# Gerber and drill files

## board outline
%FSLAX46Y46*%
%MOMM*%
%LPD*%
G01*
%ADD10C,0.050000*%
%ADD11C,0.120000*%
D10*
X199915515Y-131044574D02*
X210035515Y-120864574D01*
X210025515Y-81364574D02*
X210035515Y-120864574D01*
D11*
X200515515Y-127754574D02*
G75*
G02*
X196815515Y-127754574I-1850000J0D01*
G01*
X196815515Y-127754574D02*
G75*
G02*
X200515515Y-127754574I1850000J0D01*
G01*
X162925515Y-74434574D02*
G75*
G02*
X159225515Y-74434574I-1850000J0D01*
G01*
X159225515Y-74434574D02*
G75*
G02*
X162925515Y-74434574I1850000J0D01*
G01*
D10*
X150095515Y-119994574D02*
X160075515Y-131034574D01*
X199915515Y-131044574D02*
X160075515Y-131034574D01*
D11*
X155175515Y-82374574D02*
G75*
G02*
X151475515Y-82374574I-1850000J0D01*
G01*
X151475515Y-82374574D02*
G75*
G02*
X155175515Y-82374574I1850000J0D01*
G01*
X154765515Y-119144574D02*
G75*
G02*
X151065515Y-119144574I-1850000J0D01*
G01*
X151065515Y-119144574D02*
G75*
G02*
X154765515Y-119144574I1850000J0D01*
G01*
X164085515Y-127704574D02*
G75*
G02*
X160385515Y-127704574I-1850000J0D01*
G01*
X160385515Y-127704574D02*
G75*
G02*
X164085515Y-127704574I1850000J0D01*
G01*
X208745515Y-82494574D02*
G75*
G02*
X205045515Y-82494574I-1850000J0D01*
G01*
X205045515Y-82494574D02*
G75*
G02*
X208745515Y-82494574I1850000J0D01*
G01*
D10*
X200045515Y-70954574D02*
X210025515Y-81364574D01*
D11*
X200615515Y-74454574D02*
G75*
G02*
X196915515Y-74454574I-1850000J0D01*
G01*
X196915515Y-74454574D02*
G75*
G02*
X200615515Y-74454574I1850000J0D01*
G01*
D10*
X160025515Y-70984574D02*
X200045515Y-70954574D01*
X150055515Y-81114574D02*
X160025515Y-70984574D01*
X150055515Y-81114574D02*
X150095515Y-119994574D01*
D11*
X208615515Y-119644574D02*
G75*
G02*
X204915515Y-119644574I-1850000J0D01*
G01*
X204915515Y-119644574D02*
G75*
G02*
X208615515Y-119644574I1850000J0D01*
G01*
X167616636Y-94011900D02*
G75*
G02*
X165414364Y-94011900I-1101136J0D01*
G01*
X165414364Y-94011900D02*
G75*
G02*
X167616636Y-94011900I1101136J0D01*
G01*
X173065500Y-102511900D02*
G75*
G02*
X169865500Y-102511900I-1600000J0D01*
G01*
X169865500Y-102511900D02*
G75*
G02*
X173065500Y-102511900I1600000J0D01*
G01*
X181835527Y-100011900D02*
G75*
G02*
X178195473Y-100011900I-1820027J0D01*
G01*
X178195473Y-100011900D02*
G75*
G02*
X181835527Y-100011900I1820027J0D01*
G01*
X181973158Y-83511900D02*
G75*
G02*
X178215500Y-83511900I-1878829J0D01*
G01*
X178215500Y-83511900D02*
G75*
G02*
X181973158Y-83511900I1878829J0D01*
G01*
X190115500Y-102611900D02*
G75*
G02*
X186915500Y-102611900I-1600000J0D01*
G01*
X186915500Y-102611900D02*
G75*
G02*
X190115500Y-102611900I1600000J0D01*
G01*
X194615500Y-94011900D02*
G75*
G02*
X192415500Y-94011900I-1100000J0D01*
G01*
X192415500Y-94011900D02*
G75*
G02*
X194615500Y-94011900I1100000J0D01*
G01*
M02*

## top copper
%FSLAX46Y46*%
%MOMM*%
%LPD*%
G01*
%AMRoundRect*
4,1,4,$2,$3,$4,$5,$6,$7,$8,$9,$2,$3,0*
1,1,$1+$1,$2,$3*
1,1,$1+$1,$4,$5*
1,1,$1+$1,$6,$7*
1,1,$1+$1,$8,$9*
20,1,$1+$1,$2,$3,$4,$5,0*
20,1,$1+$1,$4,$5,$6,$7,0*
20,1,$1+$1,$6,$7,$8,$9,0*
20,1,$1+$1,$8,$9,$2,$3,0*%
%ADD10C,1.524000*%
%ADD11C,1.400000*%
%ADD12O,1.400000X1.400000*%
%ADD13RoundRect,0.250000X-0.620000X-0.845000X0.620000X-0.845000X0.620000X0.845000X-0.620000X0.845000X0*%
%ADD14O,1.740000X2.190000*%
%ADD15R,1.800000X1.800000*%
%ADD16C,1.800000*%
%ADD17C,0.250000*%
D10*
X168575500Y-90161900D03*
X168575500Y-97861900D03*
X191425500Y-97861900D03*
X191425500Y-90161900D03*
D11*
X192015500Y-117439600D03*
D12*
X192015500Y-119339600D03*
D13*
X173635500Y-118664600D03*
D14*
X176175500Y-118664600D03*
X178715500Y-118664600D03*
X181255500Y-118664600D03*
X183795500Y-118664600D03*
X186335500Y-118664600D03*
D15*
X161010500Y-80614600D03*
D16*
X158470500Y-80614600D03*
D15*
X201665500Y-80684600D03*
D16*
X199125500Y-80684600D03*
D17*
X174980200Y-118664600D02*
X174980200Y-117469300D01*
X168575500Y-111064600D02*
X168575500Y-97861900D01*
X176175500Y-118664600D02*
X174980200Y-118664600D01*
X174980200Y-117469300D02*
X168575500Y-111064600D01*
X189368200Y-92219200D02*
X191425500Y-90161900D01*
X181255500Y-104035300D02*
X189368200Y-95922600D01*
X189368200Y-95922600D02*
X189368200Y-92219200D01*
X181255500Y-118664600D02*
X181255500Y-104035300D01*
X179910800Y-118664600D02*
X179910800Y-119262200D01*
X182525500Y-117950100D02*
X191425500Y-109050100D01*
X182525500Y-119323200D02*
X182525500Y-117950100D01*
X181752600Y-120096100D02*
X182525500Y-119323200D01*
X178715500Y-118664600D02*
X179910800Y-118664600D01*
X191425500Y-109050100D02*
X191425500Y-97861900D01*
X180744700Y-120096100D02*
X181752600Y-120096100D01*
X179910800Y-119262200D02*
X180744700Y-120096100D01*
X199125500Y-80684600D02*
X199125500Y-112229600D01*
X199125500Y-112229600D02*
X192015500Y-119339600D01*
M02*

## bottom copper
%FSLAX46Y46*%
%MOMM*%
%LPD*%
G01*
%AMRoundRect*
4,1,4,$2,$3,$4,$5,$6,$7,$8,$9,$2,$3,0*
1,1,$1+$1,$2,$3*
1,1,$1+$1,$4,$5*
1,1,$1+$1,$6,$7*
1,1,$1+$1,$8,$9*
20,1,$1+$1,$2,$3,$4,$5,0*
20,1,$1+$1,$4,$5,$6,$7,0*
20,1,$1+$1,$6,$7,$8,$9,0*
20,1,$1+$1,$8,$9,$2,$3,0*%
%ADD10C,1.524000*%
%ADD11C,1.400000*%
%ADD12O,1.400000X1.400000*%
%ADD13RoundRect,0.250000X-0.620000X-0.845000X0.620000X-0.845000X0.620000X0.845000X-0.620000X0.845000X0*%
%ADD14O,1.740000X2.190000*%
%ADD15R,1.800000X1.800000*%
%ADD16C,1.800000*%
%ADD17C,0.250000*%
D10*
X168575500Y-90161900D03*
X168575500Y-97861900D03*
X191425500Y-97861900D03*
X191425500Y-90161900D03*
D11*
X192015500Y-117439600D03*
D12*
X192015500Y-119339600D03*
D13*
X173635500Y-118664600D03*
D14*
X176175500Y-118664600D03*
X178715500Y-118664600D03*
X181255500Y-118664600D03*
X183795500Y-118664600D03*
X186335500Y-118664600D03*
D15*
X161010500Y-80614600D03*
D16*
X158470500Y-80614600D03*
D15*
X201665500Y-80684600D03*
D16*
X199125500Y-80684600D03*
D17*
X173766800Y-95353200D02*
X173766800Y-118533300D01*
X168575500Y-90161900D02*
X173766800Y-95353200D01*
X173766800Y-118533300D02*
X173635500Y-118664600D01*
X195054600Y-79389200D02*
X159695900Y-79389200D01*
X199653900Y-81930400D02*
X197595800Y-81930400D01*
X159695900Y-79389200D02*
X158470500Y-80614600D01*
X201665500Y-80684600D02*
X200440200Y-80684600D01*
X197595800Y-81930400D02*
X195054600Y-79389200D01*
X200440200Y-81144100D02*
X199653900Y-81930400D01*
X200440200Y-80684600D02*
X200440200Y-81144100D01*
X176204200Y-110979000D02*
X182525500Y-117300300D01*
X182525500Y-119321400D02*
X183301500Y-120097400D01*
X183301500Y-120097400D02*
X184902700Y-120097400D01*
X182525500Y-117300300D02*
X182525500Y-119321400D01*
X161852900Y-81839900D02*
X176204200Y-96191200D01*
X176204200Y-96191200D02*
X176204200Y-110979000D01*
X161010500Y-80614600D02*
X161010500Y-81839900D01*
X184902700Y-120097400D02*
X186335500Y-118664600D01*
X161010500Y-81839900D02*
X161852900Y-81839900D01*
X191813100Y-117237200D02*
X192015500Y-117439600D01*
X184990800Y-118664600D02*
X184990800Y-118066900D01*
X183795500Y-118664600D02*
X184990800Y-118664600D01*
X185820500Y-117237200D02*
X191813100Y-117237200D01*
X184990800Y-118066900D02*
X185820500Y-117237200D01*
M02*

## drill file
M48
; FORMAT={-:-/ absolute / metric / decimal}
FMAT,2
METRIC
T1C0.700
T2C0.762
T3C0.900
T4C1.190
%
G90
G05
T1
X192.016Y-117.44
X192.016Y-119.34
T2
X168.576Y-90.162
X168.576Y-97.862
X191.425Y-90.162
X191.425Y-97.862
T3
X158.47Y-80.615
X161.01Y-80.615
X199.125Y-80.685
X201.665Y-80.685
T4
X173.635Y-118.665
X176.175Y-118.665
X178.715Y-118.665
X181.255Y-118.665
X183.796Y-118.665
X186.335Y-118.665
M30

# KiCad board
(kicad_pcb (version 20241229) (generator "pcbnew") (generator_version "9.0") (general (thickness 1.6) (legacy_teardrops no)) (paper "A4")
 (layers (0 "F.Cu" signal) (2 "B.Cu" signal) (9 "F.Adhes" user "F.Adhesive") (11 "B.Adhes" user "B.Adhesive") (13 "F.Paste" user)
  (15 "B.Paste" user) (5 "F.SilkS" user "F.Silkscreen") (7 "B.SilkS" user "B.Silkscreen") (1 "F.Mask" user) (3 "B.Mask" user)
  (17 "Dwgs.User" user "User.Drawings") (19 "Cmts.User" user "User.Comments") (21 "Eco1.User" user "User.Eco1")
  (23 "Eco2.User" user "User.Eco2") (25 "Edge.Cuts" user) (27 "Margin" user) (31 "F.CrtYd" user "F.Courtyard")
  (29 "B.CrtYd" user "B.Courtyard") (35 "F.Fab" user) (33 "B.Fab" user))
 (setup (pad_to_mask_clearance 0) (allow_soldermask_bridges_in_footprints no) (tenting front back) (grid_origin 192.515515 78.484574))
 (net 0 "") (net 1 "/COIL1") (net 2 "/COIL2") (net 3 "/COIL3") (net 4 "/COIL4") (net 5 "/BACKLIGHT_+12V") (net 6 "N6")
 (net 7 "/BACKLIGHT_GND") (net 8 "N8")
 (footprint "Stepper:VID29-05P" (layer "F.Cu") (at 180.0155 94.0119)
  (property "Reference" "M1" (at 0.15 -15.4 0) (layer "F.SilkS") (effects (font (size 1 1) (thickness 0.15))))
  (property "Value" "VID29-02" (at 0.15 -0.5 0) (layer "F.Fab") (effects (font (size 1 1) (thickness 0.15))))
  (fp_circle (center -13.5 0) (end -12.65 0.7) (stroke (width 0.12) (type solid)) (fill no) (layer "Edge.Cuts"))
  (fp_circle (center -8.55 8.5) (end -6.95 8.5) (stroke (width 0.12) (type solid)) (fill no) (layer "Edge.Cuts"))
  (fp_circle (center 0 6) (end 1.45 7.1) (stroke (width 0.12) (type solid)) (fill no) (layer "Edge.Cuts"))
  (fp_circle (center 0.078829 -10.5) (end 1.778829 -9.7) (stroke (width 0.12) (type solid)) (fill no) (layer "Edge.Cuts"))
  (fp_circle (center 8.5 8.6) (end 10.1 8.6) (stroke (width 0.12) (type solid)) (fill no) (layer "Edge.Cuts"))
  (fp_circle (center 13.5 0) (end 14.6 0) (stroke (width 0.12) (type solid)) (fill no) (layer "Edge.Cuts"))
  (pad "1" thru_hole circle (at -11.44 -3.85) (size 1.524 1.524) (drill 0.762) (layers "*.Cu" "*.Mask") (remove_unused_layers no)
   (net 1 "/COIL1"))
  (pad "2" thru_hole circle (at -11.44 3.85) (size 1.524 1.524) (drill 0.762) (layers "*.Cu" "*.Mask") (remove_unused_layers no)
   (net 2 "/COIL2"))
  (pad "3" thru_hole circle (at 11.41 3.85) (size 1.524 1.524) (drill 0.762) (layers "*.Cu" "*.Mask") (remove_unused_layers no)
   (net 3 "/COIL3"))
  (pad "4" thru_hole circle (at 11.41 -3.85) (size 1.524 1.524) (drill 0.762) (layers "*.Cu" "*.Mask") (remove_unused_layers no)
   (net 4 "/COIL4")))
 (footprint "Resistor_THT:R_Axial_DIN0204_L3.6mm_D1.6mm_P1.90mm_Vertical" (layer "F.Cu") (at 192.0155 117.4396 -90)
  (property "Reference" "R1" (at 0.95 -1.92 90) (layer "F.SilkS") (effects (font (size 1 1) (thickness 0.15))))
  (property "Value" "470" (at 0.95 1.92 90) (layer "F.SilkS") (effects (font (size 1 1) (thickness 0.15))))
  (pad "1" thru_hole circle (at 0 0 270) (size 1.4 1.4) (drill 0.7) (layers "*.Cu" "*.Mask") (remove_unused_layers no)
   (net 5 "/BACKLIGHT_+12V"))
  (pad "2" thru_hole oval (at 1.9 0 270) (size 1.4 1.4) (drill 0.7) (layers "*.Cu" "*.Mask") (remove_unused_layers no) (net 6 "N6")))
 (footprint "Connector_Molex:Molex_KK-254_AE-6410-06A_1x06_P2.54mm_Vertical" (layer "F.Cu") (at 173.6355 118.6646)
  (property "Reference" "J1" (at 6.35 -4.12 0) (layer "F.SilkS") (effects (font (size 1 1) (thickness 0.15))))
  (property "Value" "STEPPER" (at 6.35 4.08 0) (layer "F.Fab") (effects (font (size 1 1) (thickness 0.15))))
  (pad "1" thru_hole roundrect (at 0 0) (size 1.74 2.19) (drill 1.19) (layers "*.Cu" "*.Mask") (remove_unused_layers no)
   (roundrect_rratio 0.1436781609) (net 1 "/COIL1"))
  (pad "2" thru_hole oval (at 2.54 0) (size 1.74 2.19) (drill 1.19) (layers "*.Cu" "*.Mask") (remove_unused_layers no) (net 2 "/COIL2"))
  (pad "3" thru_hole oval (at 5.08 0) (size 1.74 2.19) (drill 1.19) (layers "*.Cu" "*.Mask") (remove_unused_layers no) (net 3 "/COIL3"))
  (pad "4" thru_hole oval (at 7.62 0) (size 1.74 2.19) (drill 1.19) (layers "*.Cu" "*.Mask") (remove_unused_layers no) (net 4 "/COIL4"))
  (pad "5" thru_hole oval (at 10.16 0) (size 1.74 2.19) (drill 1.19) (layers "*.Cu" "*.Mask") (remove_unused_layers no)
   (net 5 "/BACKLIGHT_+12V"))
  (pad "6" thru_hole oval (at 12.7 0) (size 1.74 2.19) (drill 1.19) (layers "*.Cu" "*.Mask") (remove_unused_layers no)
   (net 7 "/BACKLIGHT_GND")))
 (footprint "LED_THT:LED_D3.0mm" (layer "B.Cu") (at 161.0105 80.6146 180)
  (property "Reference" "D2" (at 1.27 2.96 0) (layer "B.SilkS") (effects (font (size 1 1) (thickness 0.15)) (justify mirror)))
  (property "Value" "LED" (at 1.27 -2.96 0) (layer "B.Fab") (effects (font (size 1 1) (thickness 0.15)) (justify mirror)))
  (pad "1" thru_hole rect (at 0 0 180) (size 1.8 1.8) (drill 0.9) (layers "*.Cu" "*.Mask") (remove_unused_layers no)
   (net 7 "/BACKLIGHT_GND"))
  (pad "2" thru_hole circle (at 2.54 0 180) (size 1.8 1.8) (drill 0.9) (layers "*.Cu" "*.Mask") (remove_unused_layers no) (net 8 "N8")))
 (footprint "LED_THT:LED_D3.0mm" (layer "B.Cu") (at 201.6655 80.6846 180)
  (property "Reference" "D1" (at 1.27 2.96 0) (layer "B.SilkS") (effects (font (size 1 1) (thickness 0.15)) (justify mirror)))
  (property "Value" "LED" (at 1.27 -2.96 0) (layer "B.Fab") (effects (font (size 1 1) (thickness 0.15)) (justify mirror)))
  (pad "1" thru_hole rect (at 0 0 180) (size 1.8 1.8) (drill 0.9) (layers "*.Cu" "*.Mask") (remove_unused_layers no) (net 8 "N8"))
  (pad "2" thru_hole circle (at 2.54 0 180) (size 1.8 1.8) (drill 0.9) (layers "*.Cu" "*.Mask") (remove_unused_layers no) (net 6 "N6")))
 (gr_line (start 199.915515 131.044574) (end 210.035515 120.864574) (stroke (width 0.05) (type solid)) (layer "Edge.Cuts"))
 (gr_line (start 210.025515 81.364574) (end 210.035515 120.864574) (stroke (width 0.05) (type solid)) (layer "Edge.Cuts"))
 (gr_circle (center 198.665515 127.754574) (end 200.515515 127.754574) (stroke (width 0.12) (type solid)) (fill no) (layer "Edge.Cuts"))
 (gr_circle (center 161.075515 74.434574) (end 162.925515 74.434574) (stroke (width 0.12) (type solid)) (fill no) (layer "Edge.Cuts"))
 (gr_line (start 150.095515 119.994574) (end 160.075515 131.034574) (stroke (width 0.05) (type solid)) (layer "Edge.Cuts"))
 (gr_line (start 199.915515 131.044574) (end 160.075515 131.034574) (stroke (width 0.05) (type solid)) (layer "Edge.Cuts"))
 (gr_circle (center 153.325515 82.374574) (end 155.175515 82.374574) (stroke (width 0.12) (type solid)) (fill no) (layer "Edge.Cuts"))
 (gr_circle (center 152.915515 119.144574) (end 154.765515 119.144574) (stroke (width 0.12) (type solid)) (fill no) (layer "Edge.Cuts"))
 (gr_circle (center 162.235515 127.704574) (end 164.085515 127.704574) (stroke (width 0.12) (type solid)) (fill no) (layer "Edge.Cuts"))
 (gr_circle (center 206.895515 82.494574) (end 208.745515 82.494574) (stroke (width 0.12) (type solid)) (fill no) (layer "Edge.Cuts"))
 (gr_line (start 200.045515 70.954574) (end 210.025515 81.364574) (stroke (width 0.05) (type solid)) (layer "Edge.Cuts"))
 (gr_circle (center 198.765515 74.454574) (end 200.615515 74.454574) (stroke (width 0.12) (type solid)) (fill no) (layer "Edge.Cuts"))
 (gr_line (start 160.025515 70.984574) (end 200.045515 70.954574) (stroke (width 0.05) (type solid)) (layer "Edge.Cuts"))
 (gr_line (start 150.055515 81.114574) (end 160.025515 70.984574) (stroke (width 0.05) (type solid)) (layer "Edge.Cuts"))
 (gr_line (start 150.055515 81.114574) (end 150.095515 119.994574) (stroke (width 0.05) (type solid)) (layer "Edge.Cuts"))
 (gr_circle (center 206.765515 119.644574) (end 208.615515 119.644574) (stroke (width 0.12) (type solid)) (fill no) (layer "Edge.Cuts"))
 (segment (start 174.9802 118.6646) (end 174.9802 117.4693) (width 0.25) (layer "F.Cu") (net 2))
 (segment (start 168.5755 111.0646) (end 168.5755 97.8619) (width 0.25) (layer "F.Cu") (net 2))
 (segment (start 176.1755 118.6646) (end 174.9802 118.6646) (width 0.25) (layer "F.Cu") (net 2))
 (segment (start 174.9802 117.4693) (end 168.5755 111.0646) (width 0.25) (layer "F.Cu") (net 2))
 (segment (start 173.7668 95.3532) (end 173.7668 118.5333) (width 0.25) (layer "B.Cu") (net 1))
 (segment (start 168.5755 90.1619) (end 173.7668 95.3532) (width 0.25) (layer "B.Cu") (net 1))
 (segment (start 173.7668 118.5333) (end 173.6355 118.6646) (width 0.25) (layer "B.Cu") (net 1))
 (segment (start 189.3682 92.2192) (end 191.4255 90.1619) (width 0.25) (layer "F.Cu") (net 4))
 (segment (start 181.2555 104.0353) (end 189.3682 95.9226) (width 0.25) (layer "F.Cu") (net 4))
 (segment (start 189.3682 95.9226) (end 189.3682 92.2192) (width 0.25) (layer "F.Cu") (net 4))
 (segment (start 181.2555 118.6646) (end 181.2555 104.0353) (width 0.25) (layer "F.Cu") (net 4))
 (segment (start 179.9108 118.6646) (end 179.9108 119.2622) (width 0.25) (layer "F.Cu") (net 3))
 (segment (start 182.5255 117.9501) (end 191.4255 109.0501) (width 0.25) (layer "F.Cu") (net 3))
 (segment (start 182.5255 119.3232) (end 182.5255 117.9501) (width 0.25) (layer "F.Cu") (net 3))
 (segment (start 181.7526 120.0961) (end 182.5255 119.3232) (width 0.25) (layer "F.Cu") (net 3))
 (segment (start 178.7155 118.6646) (end 179.9108 118.6646) (width 0.25) (layer "F.Cu") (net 3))
 (segment (start 191.4255 109.0501) (end 191.4255 97.8619) (width 0.25) (layer "F.Cu") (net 3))
 (segment (start 180.7447 120.0961) (end 181.7526 120.0961) (width 0.25) (layer "F.Cu") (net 3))
 (segment (start 179.9108 119.2622) (end 180.7447 120.0961) (width 0.25) (layer "F.Cu") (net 3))
 (segment (start 195.0546 79.3892) (end 159.6959 79.3892) (width 0.25) (layer "B.Cu") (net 8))
 (segment (start 199.6539 81.9304) (end 197.5958 81.9304) (width 0.25) (layer "B.Cu") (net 8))
 (segment (start 159.6959 79.3892) (end 158.4705 80.6146) (width 0.25) (layer "B.Cu") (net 8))
 (segment (start 201.6655 80.6846) (end 200.4402 80.6846) (width 0.25) (layer "B.Cu") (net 8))
 (segment (start 197.5958 81.9304) (end 195.0546 79.3892) (width 0.25) (layer "B.Cu") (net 8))
 (segment (start 200.4402 81.1441) (end 199.6539 81.9304) (width 0.25) (layer "B.Cu") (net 8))
 (segment (start 200.4402 80.6846) (end 200.4402 81.1441) (width 0.25) (layer "B.Cu") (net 8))
 (segment (start 199.1255 80.6846) (end 199.1255 112.2296) (width 0.25) (layer "F.Cu") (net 6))
 (segment (start 199.1255 112.2296) (end 192.0155 119.3396) (width 0.25) (layer "F.Cu") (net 6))
 (segment (start 176.2042 110.979) (end 182.5255 117.3003) (width 0.25) (layer "B.Cu") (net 7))
 (segment (start 182.5255 119.3214) (end 183.3015 120.0974) (width 0.25) (layer "B.Cu") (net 7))
 (segment (start 183.3015 120.0974) (end 184.9027 120.0974) (width 0.25) (layer "B.Cu") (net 7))
 (segment (start 182.5255 117.3003) (end 182.5255 119.3214) (width 0.25) (layer "B.Cu") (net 7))
 (segment (start 161.8529 81.8399) (end 176.2042 96.1912) (width 0.25) (layer "B.Cu") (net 7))
 (segment (start 176.2042 96.1912) (end 176.2042 110.979) (width 0.25) (layer "B.Cu") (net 7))
 (segment (start 161.0105 80.6146) (end 161.0105 81.8399) (width 0.25) (layer "B.Cu") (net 7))
 (segment (start 184.9027 120.0974) (end 186.3355 118.6646) (width 0.25) (layer "B.Cu") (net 7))
 (segment (start 161.0105 81.8399) (end 161.8529 81.8399) (width 0.25) (layer "B.Cu") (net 7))
 (segment (start 191.8131 117.2372) (end 192.0155 117.4396) (width 0.25) (layer "B.Cu") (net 5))
 (segment (start 184.9908 118.6646) (end 184.9908 118.0669) (width 0.25) (layer "B.Cu") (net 5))
 (segment (start 183.7955 118.6646) (end 184.9908 118.6646) (width 0.25) (layer "B.Cu") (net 5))
 (segment (start 185.8205 117.2372) (end 191.8131 117.2372) (width 0.25) (layer "B.Cu") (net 5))
 (segment (start 184.9908 118.0669) (end 185.8205 117.2372) (width 0.25) (layer "B.Cu") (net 5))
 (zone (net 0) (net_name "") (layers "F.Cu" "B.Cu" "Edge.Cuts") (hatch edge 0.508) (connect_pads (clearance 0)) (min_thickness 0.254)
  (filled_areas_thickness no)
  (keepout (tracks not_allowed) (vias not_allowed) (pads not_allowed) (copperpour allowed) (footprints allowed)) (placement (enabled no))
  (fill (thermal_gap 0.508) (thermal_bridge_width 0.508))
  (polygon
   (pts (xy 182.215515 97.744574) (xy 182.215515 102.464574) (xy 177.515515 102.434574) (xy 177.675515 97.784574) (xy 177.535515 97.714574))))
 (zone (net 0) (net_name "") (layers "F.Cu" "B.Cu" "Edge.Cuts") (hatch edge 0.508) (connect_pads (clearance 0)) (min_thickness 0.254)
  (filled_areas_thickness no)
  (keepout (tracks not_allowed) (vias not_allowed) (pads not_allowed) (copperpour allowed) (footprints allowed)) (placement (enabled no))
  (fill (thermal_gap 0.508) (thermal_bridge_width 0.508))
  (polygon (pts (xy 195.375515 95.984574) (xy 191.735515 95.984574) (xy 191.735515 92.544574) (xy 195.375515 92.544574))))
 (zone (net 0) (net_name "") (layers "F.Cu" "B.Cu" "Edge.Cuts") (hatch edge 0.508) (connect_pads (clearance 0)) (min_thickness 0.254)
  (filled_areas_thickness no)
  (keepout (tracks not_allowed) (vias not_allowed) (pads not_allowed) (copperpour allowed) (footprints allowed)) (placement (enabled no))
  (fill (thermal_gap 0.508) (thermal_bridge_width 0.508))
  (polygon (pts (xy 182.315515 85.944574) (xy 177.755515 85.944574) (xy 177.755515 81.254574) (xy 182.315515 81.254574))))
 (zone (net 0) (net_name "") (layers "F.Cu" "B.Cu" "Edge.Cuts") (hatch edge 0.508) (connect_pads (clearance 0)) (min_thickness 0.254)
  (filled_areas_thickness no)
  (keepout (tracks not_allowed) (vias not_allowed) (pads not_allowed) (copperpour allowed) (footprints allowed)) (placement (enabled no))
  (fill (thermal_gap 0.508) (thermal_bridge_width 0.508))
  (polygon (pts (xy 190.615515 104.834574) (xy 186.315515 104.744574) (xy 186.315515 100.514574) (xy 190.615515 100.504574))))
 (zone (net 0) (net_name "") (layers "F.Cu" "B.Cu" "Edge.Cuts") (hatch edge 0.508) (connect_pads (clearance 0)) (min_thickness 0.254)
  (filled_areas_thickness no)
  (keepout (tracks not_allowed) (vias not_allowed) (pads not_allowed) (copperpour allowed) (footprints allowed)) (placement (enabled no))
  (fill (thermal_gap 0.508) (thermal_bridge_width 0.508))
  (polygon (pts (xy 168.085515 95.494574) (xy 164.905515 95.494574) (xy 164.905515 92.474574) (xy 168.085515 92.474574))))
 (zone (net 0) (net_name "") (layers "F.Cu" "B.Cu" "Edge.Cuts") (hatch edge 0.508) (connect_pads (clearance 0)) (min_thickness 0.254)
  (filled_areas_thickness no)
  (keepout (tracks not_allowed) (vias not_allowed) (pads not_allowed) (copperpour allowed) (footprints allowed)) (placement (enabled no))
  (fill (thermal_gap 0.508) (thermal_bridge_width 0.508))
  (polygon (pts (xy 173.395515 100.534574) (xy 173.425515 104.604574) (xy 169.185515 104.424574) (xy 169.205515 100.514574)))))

